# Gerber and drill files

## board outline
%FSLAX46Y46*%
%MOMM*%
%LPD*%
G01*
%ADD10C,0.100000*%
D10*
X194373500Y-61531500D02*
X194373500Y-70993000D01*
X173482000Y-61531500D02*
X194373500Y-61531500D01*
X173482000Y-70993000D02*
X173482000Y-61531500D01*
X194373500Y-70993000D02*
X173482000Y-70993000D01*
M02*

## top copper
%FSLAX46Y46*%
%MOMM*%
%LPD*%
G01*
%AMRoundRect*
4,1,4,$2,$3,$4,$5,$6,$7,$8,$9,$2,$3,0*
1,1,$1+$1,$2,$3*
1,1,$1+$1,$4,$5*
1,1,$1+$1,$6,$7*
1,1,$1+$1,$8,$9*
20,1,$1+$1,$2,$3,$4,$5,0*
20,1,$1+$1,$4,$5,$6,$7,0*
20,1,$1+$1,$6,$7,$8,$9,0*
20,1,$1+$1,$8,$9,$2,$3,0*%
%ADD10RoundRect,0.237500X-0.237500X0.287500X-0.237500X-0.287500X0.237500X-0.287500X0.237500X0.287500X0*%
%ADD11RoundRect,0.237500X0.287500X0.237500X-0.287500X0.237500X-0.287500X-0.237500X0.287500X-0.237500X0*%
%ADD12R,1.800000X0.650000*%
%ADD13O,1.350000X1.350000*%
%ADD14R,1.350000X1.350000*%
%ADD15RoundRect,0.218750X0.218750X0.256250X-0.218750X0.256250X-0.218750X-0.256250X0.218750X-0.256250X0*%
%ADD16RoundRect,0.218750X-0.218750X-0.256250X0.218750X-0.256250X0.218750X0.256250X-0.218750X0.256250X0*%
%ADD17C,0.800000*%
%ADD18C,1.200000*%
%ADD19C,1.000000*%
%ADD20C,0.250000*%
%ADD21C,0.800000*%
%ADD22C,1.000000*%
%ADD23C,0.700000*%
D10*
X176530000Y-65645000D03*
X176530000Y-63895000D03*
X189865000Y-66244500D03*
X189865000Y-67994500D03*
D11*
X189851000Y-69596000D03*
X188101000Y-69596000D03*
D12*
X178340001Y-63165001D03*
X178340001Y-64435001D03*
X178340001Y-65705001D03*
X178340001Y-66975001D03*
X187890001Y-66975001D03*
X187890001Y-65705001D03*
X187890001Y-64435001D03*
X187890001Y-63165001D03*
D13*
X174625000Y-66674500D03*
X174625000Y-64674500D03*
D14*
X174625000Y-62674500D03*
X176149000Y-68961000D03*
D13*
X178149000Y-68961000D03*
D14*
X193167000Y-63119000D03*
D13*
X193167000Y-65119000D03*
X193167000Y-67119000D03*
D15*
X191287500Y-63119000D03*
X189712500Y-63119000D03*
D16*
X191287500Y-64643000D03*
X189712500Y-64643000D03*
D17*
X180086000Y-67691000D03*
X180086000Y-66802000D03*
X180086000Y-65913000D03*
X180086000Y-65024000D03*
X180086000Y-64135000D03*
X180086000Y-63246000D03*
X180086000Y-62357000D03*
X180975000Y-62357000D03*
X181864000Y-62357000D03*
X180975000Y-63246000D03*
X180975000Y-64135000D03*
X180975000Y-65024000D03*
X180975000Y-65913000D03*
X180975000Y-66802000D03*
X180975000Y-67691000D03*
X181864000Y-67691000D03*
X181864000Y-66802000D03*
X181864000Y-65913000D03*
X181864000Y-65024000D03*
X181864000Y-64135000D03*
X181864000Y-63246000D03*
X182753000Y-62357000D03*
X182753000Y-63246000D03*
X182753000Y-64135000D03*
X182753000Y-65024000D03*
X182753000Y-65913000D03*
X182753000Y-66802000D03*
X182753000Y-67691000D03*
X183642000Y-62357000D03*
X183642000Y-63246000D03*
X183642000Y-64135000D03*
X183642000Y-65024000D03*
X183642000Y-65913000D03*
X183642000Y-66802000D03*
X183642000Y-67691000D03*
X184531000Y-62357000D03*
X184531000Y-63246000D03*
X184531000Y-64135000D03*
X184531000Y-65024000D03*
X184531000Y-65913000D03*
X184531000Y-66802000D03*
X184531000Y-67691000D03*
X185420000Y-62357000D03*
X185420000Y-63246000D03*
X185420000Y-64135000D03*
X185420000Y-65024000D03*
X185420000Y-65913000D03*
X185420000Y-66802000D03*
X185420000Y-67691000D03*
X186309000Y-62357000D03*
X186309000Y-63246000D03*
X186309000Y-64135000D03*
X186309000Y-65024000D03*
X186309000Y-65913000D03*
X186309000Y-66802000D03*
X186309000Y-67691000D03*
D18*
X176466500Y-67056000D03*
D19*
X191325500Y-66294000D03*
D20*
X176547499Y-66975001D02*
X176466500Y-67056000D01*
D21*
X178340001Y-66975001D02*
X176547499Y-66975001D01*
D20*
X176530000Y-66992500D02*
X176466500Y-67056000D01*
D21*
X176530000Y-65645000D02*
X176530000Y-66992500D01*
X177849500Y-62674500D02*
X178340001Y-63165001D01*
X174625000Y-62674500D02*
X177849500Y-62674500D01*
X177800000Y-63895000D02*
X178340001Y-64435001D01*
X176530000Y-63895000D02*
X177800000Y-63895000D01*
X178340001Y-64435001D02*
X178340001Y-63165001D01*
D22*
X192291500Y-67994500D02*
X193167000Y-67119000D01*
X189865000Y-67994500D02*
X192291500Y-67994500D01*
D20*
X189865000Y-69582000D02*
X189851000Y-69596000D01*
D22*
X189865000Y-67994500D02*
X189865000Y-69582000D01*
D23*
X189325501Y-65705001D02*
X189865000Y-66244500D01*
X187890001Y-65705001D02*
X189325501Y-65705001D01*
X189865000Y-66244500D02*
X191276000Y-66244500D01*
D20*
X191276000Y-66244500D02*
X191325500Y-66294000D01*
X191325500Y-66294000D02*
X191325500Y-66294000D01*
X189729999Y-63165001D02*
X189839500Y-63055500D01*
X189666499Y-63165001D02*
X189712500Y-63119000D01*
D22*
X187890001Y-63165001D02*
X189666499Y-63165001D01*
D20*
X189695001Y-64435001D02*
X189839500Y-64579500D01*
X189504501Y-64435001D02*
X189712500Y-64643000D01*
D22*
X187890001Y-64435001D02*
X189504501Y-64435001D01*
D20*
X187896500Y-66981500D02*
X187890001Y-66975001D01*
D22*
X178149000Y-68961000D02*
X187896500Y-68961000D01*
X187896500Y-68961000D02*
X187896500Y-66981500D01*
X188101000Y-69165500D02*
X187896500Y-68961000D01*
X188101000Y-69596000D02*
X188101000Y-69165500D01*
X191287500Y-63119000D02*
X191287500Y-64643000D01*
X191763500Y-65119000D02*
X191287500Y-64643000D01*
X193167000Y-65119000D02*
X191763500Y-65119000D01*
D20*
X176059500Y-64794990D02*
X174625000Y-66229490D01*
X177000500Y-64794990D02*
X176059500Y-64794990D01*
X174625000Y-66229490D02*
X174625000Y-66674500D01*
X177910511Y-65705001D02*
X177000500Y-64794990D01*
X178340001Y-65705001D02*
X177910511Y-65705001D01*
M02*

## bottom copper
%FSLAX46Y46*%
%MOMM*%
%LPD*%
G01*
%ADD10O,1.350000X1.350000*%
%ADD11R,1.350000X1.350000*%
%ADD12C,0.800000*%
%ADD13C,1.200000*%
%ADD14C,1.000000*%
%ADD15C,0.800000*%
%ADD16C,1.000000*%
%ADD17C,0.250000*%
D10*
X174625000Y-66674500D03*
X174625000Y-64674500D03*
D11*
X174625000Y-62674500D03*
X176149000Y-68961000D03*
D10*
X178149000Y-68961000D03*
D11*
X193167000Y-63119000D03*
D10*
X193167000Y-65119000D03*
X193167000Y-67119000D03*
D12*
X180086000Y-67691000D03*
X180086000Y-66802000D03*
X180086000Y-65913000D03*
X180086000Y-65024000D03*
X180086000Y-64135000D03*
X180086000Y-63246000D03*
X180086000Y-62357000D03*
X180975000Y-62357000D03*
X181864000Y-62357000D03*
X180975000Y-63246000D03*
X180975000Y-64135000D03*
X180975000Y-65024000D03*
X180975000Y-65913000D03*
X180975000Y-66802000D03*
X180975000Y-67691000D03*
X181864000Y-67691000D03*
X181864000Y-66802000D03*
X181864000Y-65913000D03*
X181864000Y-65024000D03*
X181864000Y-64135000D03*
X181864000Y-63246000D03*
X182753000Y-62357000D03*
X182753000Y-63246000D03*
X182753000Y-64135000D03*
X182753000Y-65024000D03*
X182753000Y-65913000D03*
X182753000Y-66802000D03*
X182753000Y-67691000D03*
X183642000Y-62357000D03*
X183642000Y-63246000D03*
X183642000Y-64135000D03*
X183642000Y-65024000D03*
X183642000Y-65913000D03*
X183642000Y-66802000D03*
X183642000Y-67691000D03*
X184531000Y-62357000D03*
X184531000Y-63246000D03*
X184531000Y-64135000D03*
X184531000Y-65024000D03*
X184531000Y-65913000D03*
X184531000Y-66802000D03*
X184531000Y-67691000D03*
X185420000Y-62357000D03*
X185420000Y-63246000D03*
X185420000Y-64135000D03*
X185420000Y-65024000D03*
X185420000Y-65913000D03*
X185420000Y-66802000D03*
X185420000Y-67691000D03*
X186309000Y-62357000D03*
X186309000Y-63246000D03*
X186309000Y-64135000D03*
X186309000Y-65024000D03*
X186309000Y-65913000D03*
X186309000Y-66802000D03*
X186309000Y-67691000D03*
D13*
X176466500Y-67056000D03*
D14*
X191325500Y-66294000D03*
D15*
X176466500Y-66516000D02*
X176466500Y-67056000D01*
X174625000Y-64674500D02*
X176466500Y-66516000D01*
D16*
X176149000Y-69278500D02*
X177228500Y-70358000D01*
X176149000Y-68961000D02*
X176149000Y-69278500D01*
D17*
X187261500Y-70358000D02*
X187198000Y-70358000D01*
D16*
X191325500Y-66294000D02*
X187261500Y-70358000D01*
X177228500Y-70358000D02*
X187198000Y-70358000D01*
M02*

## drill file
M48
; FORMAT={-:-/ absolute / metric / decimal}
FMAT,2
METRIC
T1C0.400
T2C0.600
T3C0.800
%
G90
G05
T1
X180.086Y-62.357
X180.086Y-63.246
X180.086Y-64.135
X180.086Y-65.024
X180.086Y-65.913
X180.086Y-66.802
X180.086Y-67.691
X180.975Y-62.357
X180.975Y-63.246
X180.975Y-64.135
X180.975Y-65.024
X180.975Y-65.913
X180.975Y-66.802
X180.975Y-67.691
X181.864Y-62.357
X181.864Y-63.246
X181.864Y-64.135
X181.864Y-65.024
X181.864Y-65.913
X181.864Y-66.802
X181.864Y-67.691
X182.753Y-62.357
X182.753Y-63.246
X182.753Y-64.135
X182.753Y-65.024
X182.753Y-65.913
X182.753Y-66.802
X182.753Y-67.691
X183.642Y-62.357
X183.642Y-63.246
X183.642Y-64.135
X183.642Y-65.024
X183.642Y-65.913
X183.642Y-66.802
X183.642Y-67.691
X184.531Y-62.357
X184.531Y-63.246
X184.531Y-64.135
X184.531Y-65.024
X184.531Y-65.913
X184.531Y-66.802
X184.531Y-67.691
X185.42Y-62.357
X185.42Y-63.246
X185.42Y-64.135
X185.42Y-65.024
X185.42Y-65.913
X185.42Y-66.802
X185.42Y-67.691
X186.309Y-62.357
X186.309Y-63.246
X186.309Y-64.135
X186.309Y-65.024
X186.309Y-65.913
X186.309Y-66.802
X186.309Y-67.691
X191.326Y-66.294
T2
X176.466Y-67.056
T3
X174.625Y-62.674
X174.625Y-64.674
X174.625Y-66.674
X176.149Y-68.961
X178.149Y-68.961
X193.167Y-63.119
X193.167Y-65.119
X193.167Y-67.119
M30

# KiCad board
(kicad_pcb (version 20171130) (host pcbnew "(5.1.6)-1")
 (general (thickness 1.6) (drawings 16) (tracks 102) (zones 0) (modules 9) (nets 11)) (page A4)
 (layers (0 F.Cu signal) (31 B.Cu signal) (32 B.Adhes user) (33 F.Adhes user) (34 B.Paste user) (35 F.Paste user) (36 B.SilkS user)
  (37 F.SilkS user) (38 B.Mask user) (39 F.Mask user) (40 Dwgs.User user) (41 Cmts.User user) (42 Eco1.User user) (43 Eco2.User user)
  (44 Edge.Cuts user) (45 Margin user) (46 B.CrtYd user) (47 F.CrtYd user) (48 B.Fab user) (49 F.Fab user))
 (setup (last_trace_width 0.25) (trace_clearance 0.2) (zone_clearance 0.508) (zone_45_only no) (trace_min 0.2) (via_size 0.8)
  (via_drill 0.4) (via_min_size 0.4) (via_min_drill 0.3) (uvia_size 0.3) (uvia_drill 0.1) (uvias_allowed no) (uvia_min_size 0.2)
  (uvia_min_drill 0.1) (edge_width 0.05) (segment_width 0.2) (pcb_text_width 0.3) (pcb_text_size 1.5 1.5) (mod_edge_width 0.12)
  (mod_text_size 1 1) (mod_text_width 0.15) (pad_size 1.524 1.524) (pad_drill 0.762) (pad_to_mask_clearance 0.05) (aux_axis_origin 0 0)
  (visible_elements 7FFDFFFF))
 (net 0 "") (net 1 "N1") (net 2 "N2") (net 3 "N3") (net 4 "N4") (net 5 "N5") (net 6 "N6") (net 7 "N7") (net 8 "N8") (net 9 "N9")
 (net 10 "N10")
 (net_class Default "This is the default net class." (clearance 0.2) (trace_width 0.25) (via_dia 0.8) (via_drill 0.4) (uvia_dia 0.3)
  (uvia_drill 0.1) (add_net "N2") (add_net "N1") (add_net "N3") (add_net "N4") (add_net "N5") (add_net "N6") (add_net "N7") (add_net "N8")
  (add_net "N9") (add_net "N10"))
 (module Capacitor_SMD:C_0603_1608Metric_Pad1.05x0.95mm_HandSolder (layer F.Cu) (at 176.53 64.77 270)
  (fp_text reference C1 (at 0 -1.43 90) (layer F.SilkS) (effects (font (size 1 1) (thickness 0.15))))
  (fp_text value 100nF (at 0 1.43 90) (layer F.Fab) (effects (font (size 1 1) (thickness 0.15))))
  (pad 2 smd roundrect (at 0.875 0 270) (size 1.05 0.95) (layers F.Cu F.Paste F.Mask) (roundrect_rratio 0.25) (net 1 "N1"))
  (pad 1 smd roundrect (at -0.875 0 270) (size 1.05 0.95) (layers F.Cu F.Paste F.Mask) (roundrect_rratio 0.25) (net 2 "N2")))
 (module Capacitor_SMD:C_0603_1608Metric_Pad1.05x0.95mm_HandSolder (layer F.Cu) (at 189.865 67.1195 270)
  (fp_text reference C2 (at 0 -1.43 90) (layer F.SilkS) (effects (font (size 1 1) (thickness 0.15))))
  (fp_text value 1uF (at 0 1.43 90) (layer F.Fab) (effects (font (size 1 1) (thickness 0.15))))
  (pad 1 smd roundrect (at -0.875 0 270) (size 1.05 0.95) (layers F.Cu F.Paste F.Mask) (roundrect_rratio 0.25) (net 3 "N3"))
  (pad 2 smd roundrect (at 0.875 0 270) (size 1.05 0.95) (layers F.Cu F.Paste F.Mask) (roundrect_rratio 0.25) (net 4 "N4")))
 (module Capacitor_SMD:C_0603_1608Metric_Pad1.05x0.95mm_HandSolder (layer F.Cu) (at 188.976 69.596 180)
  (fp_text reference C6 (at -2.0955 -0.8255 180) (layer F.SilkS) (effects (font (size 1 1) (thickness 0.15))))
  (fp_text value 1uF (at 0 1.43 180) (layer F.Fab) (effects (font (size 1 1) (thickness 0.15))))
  (pad 1 smd roundrect (at -0.875 0 180) (size 1.05 0.95) (layers F.Cu F.Paste F.Mask) (roundrect_rratio 0.25) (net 4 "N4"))
  (pad 2 smd roundrect (at 0.875 0 180) (size 1.05 0.95) (layers F.Cu F.Paste F.Mask) (roundrect_rratio 0.25) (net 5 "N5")))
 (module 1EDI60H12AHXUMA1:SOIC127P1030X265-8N (layer F.Cu) (at 183.115001 65.070001)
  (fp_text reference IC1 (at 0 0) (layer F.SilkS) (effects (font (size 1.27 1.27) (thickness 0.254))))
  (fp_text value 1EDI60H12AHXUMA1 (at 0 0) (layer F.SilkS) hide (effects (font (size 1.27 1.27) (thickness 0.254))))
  (pad 1 smd rect (at -4.775 -1.905 90) (size 0.65 1.8) (layers F.Cu F.Paste F.Mask) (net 2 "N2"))
  (pad 2 smd rect (at -4.775 -0.635 90) (size 0.65 1.8) (layers F.Cu F.Paste F.Mask) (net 2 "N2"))
  (pad 3 smd rect (at -4.775 0.635 90) (size 0.65 1.8) (layers F.Cu F.Paste F.Mask) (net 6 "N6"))
  (pad 4 smd rect (at -4.775 1.905 90) (size 0.65 1.8) (layers F.Cu F.Paste F.Mask) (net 1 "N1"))
  (pad 5 smd rect (at 4.775 1.905 90) (size 0.65 1.8) (layers F.Cu F.Paste F.Mask) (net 5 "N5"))
  (pad 6 smd rect (at 4.775 0.635 90) (size 0.65 1.8) (layers F.Cu F.Paste F.Mask) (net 3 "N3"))
  (pad 7 smd rect (at 4.775 -0.635 90) (size 0.65 1.8) (layers F.Cu F.Paste F.Mask) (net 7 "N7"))
  (pad 8 smd rect (at 4.775 -1.905 90) (size 0.65 1.8) (layers F.Cu F.Paste F.Mask) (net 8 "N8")))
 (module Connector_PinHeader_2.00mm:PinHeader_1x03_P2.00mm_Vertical (layer B.Cu) (at 174.625 62.6745 180)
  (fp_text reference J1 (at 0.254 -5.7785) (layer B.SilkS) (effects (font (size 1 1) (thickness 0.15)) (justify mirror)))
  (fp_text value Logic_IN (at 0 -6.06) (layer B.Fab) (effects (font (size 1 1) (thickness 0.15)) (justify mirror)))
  (pad 3 thru_hole oval (at 0 -4 180) (size 1.35 1.35) (drill 0.8) (layers *.Cu *.Mask) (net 6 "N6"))
  (pad 2 thru_hole oval (at 0 -2 180) (size 1.35 1.35) (drill 0.8) (layers *.Cu *.Mask) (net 1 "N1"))
  (pad 1 thru_hole rect (at 0 0 180) (size 1.35 1.35) (drill 0.8) (layers *.Cu *.Mask) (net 2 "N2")))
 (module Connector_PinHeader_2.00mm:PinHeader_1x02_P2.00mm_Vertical (layer B.Cu) (at 176.149 68.961 270)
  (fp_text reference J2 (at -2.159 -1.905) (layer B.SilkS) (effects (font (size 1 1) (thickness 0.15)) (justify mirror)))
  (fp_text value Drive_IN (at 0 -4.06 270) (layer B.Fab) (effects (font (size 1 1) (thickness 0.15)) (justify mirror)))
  (pad 1 thru_hole rect (at 0 0 270) (size 1.35 1.35) (drill 0.8) (layers *.Cu *.Mask) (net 3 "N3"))
  (pad 2 thru_hole oval (at 0 -2 270) (size 1.35 1.35) (drill 0.8) (layers *.Cu *.Mask) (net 5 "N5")))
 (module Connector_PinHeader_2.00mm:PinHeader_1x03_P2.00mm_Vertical (layer B.Cu) (at 193.167 63.119 180)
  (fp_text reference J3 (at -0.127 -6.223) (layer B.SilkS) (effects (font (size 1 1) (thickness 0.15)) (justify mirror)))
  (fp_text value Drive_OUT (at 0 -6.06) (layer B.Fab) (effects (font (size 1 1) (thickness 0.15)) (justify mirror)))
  (pad 1 thru_hole rect (at 0 0 180) (size 1.35 1.35) (drill 0.8) (layers *.Cu *.Mask) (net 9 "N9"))
  (pad 2 thru_hole oval (at 0 -2 180) (size 1.35 1.35) (drill 0.8) (layers *.Cu *.Mask) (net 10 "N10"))
  (pad 3 thru_hole oval (at 0 -4 180) (size 1.35 1.35) (drill 0.8) (layers *.Cu *.Mask) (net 4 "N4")))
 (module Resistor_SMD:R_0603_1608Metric (layer F.Cu) (at 190.5 63.119 180)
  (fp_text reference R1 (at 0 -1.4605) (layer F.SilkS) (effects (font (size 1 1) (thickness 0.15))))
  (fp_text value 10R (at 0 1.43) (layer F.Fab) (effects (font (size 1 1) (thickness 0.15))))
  (pad 1 smd roundrect (at -0.7875 0 180) (size 0.875 0.95) (layers F.Cu F.Paste F.Mask) (roundrect_rratio 0.25) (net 10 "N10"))
  (pad 2 smd roundrect (at 0.7875 0 180) (size 0.875 0.95) (layers F.Cu F.Paste F.Mask) (roundrect_rratio 0.25) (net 8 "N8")))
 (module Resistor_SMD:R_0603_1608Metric (layer F.Cu) (at 190.5 64.643)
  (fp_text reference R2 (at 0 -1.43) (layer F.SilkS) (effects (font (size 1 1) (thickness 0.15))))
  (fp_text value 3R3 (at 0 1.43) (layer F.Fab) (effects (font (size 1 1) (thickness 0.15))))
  (pad 2 smd roundrect (at 0.7875 0) (size 0.875 0.95) (layers F.Cu F.Paste F.Mask) (roundrect_rratio 0.25) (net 10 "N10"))
  (pad 1 smd roundrect (at -0.7875 0) (size 0.875 0.95) (layers F.Cu F.Paste F.Mask) (roundrect_rratio 0.25) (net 7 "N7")))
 (gr_line (start 194.3735 61.5315) (end 194.3735 70.993) (layer Edge.Cuts) (width 0.1))
 (gr_line (start 173.482 61.5315) (end 194.3735 61.5315) (layer Edge.Cuts) (width 0.1))
 (gr_line (start 173.482 70.993) (end 173.482 61.5315) (layer Edge.Cuts) (width 0.1))
 (gr_line (start 194.3735 70.993) (end 173.482 70.993) (layer Edge.Cuts) (width 0.1))
 (via (at 180.086 67.691) (size 0.8) (drill 0.4) (layers F.Cu B.Cu) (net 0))
 (via (at 180.086 66.802) (size 0.8) (drill 0.4) (layers F.Cu B.Cu) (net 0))
 (via (at 180.086 65.913) (size 0.8) (drill 0.4) (layers F.Cu B.Cu) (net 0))
 (via (at 180.086 65.024) (size 0.8) (drill 0.4) (layers F.Cu B.Cu) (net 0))
 (via (at 180.086 64.135) (size 0.8) (drill 0.4) (layers F.Cu B.Cu) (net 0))
 (via (at 180.086 63.246) (size 0.8) (drill 0.4) (layers F.Cu B.Cu) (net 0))
 (via (at 180.086 62.357) (size 0.8) (drill 0.4) (layers F.Cu B.Cu) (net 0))
 (via (at 180.975 62.357) (size 0.8) (drill 0.4) (layers F.Cu B.Cu) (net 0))
 (via (at 181.864 62.357) (size 0.8) (drill 0.4) (layers F.Cu B.Cu) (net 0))
 (via (at 180.975 63.246) (size 0.8) (drill 0.4) (layers F.Cu B.Cu) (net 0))
 (via (at 180.975 64.135) (size 0.8) (drill 0.4) (layers F.Cu B.Cu) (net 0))
 (via (at 180.975 65.024) (size 0.8) (drill 0.4) (layers F.Cu B.Cu) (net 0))
 (via (at 180.975 65.913) (size 0.8) (drill 0.4) (layers F.Cu B.Cu) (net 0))
 (via (at 180.975 66.802) (size 0.8) (drill 0.4) (layers F.Cu B.Cu) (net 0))
 (via (at 180.975 67.691) (size 0.8) (drill 0.4) (layers F.Cu B.Cu) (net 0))
 (via (at 181.864 67.691) (size 0.8) (drill 0.4) (layers F.Cu B.Cu) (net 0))
 (via (at 181.864 66.802) (size 0.8) (drill 0.4) (layers F.Cu B.Cu) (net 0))
 (via (at 181.864 65.913) (size 0.8) (drill 0.4) (layers F.Cu B.Cu) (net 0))
 (via (at 181.864 65.024) (size 0.8) (drill 0.4) (layers F.Cu B.Cu) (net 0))
 (via (at 181.864 64.135) (size 0.8) (drill 0.4) (layers F.Cu B.Cu) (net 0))
 (via (at 181.864 63.246) (size 0.8) (drill 0.4) (layers F.Cu B.Cu) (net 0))
 (via (at 182.753 62.357) (size 0.8) (drill 0.4) (layers F.Cu B.Cu) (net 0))
 (via (at 182.753 63.246) (size 0.8) (drill 0.4) (layers F.Cu B.Cu) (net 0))
 (via (at 182.753 64.135) (size 0.8) (drill 0.4) (layers F.Cu B.Cu) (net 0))
 (via (at 182.753 65.024) (size 0.8) (drill 0.4) (layers F.Cu B.Cu) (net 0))
 (via (at 182.753 65.913) (size 0.8) (drill 0.4) (layers F.Cu B.Cu) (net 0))
 (via (at 182.753 66.802) (size 0.8) (drill 0.4) (layers F.Cu B.Cu) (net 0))
 (via (at 182.753 67.691) (size 0.8) (drill 0.4) (layers F.Cu B.Cu) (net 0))
 (via (at 183.642 62.357) (size 0.8) (drill 0.4) (layers F.Cu B.Cu) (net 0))
 (via (at 183.642 63.246) (size 0.8) (drill 0.4) (layers F.Cu B.Cu) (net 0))
 (via (at 183.642 64.135) (size 0.8) (drill 0.4) (layers F.Cu B.Cu) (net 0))
 (via (at 183.642 65.024) (size 0.8) (drill 0.4) (layers F.Cu B.Cu) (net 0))
 (via (at 183.642 65.913) (size 0.8) (drill 0.4) (layers F.Cu B.Cu) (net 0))
 (via (at 183.642 66.802) (size 0.8) (drill 0.4) (layers F.Cu B.Cu) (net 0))
 (via (at 183.642 67.691) (size 0.8) (drill 0.4) (layers F.Cu B.Cu) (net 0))
 (via (at 184.531 62.357) (size 0.8) (drill 0.4) (layers F.Cu B.Cu) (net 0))
 (via (at 184.531 63.246) (size 0.8) (drill 0.4) (layers F.Cu B.Cu) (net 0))
 (via (at 184.531 64.135) (size 0.8) (drill 0.4) (layers F.Cu B.Cu) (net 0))
 (via (at 184.531 65.024) (size 0.8) (drill 0.4) (layers F.Cu B.Cu) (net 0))
 (via (at 184.531 65.913) (size 0.8) (drill 0.4) (layers F.Cu B.Cu) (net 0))
 (via (at 184.531 66.802) (size 0.8) (drill 0.4) (layers F.Cu B.Cu) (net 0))
 (via (at 184.531 67.691) (size 0.8) (drill 0.4) (layers F.Cu B.Cu) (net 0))
 (via (at 185.42 62.357) (size 0.8) (drill 0.4) (layers F.Cu B.Cu) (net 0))
 (via (at 185.42 63.246) (size 0.8) (drill 0.4) (layers F.Cu B.Cu) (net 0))
 (via (at 185.42 64.135) (size 0.8) (drill 0.4) (layers F.Cu B.Cu) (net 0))
 (via (at 185.42 65.024) (size 0.8) (drill 0.4) (layers F.Cu B.Cu) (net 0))
 (via (at 185.42 65.913) (size 0.8) (drill 0.4) (layers F.Cu B.Cu) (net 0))
 (via (at 185.42 66.802) (size 0.8) (drill 0.4) (layers F.Cu B.Cu) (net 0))
 (via (at 185.42 67.691) (size 0.8) (drill 0.4) (layers F.Cu B.Cu) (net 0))
 (via (at 186.309 62.357) (size 0.8) (drill 0.4) (layers F.Cu B.Cu) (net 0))
 (via (at 186.309 63.246) (size 0.8) (drill 0.4) (layers F.Cu B.Cu) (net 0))
 (via (at 186.309 64.135) (size 0.8) (drill 0.4) (layers F.Cu B.Cu) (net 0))
 (via (at 186.309 65.024) (size 0.8) (drill 0.4) (layers F.Cu B.Cu) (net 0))
 (via (at 186.309 65.913) (size 0.8) (drill 0.4) (layers F.Cu B.Cu) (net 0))
 (via (at 186.309 66.802) (size 0.8) (drill 0.4) (layers F.Cu B.Cu) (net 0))
 (via (at 186.309 67.691) (size 0.8) (drill 0.4) (layers F.Cu B.Cu) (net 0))
 (via (at 176.4665 67.056) (size 1.2) (drill 0.6) (layers F.Cu B.Cu) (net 1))
 (segment (start 176.547499 66.975001) (end 176.4665 67.056) (width 0.25) (layer F.Cu) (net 1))
 (segment (start 178.340001 66.975001) (end 176.547499 66.975001) (width 0.8) (layer F.Cu) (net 1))
 (segment (start 176.53 66.9925) (end 176.4665 67.056) (width 0.25) (layer F.Cu) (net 1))
 (segment (start 176.53 65.645) (end 176.53 66.9925) (width 0.8) (layer F.Cu) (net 1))
 (segment (start 176.4665 66.516) (end 176.4665 67.056) (width 0.8) (layer B.Cu) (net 1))
 (segment (start 174.625 64.6745) (end 176.4665 66.516) (width 0.8) (layer B.Cu) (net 1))
 (segment (start 177.8495 62.6745) (end 178.340001 63.165001) (width 0.8) (layer F.Cu) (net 2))
 (segment (start 174.625 62.6745) (end 177.8495 62.6745) (width 0.8) (layer F.Cu) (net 2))
 (segment (start 177.8 63.895) (end 178.340001 64.435001) (width 0.8) (layer F.Cu) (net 2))
 (segment (start 176.53 63.895) (end 177.8 63.895) (width 0.8) (layer F.Cu) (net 2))
 (segment (start 178.340001 64.435001) (end 178.340001 63.165001) (width 0.8) (layer F.Cu) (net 2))
 (segment (start 192.2915 67.9945) (end 193.167 67.119) (width 1) (layer F.Cu) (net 4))
 (segment (start 189.865 67.9945) (end 192.2915 67.9945) (width 1) (layer F.Cu) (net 4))
 (segment (start 189.865 69.582) (end 189.851 69.596) (width 0.25) (layer F.Cu) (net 4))
 (segment (start 189.865 67.9945) (end 189.865 69.582) (width 1) (layer F.Cu) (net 4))
 (segment (start 189.325501 65.705001) (end 189.865 66.2445) (width 0.7) (layer F.Cu) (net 3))
 (segment (start 187.890001 65.705001) (end 189.325501 65.705001) (width 0.7) (layer F.Cu) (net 3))
 (segment (start 189.865 66.2445) (end 191.276 66.2445) (width 0.7) (layer F.Cu) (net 3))
 (segment (start 191.276 66.2445) (end 191.3255 66.294) (width 0.25) (layer F.Cu) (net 3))
 (segment (start 191.3255 66.294) (end 191.3255 66.294) (width 0.25) (layer F.Cu) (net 3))
 (via (at 191.3255 66.294) (size 1) (drill 0.4) (layers F.Cu B.Cu) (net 3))
 (segment (start 176.149 69.2785) (end 177.2285 70.358) (width 1) (layer B.Cu) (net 3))
 (segment (start 176.149 68.961) (end 176.149 69.2785) (width 1) (layer B.Cu) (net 3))
 (segment (start 187.2615 70.358) (end 187.198 70.358) (width 0.25) (layer B.Cu) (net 3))
 (segment (start 191.3255 66.294) (end 187.2615 70.358) (width 1) (layer B.Cu) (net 3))
 (segment (start 177.2285 70.358) (end 187.198 70.358) (width 1) (layer B.Cu) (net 3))
 (segment (start 189.729999 63.165001) (end 189.8395 63.0555) (width 0.25) (layer F.Cu) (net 8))
 (segment (start 189.666499 63.165001) (end 189.7125 63.119) (width 0.25) (layer F.Cu) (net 8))
 (segment (start 187.890001 63.165001) (end 189.666499 63.165001) (width 1) (layer F.Cu) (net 8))
 (segment (start 189.695001 64.435001) (end 189.8395 64.5795) (width 0.25) (layer F.Cu) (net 7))
 (segment (start 189.504501 64.435001) (end 189.7125 64.643) (width 0.25) (layer F.Cu) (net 7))
 (segment (start 187.890001 64.435001) (end 189.504501 64.435001) (width 1) (layer F.Cu) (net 7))
 (segment (start 187.8965 66.9815) (end 187.890001 66.975001) (width 0.25) (layer F.Cu) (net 5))
 (segment (start 178.149 68.961) (end 187.8965 68.961) (width 1) (layer F.Cu) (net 5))
 (segment (start 187.8965 68.961) (end 187.8965 66.9815) (width 1) (layer F.Cu) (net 5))
 (segment (start 188.101 69.1655) (end 187.8965 68.961) (width 1) (layer F.Cu) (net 5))
 (segment (start 188.101 69.596) (end 188.101 69.1655) (width 1) (layer F.Cu) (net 5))
 (segment (start 191.2875 63.119) (end 191.2875 64.643) (width 1) (layer F.Cu) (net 10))
 (segment (start 191.7635 65.119) (end 191.2875 64.643) (width 1) (layer F.Cu) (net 10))
 (segment (start 193.167 65.119) (end 191.7635 65.119) (width 1) (layer F.Cu) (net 10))
 (segment (start 176.0595 64.79499) (end 174.625 66.22949) (width 0.25) (layer F.Cu) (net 6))
 (segment (start 177.0005 64.79499) (end 176.0595 64.79499) (width 0.25) (layer F.Cu) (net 6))
 (segment (start 174.625 66.22949) (end 174.625 66.6745) (width 0.25) (layer F.Cu) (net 6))
 (segment (start 177.910511 65.705001) (end 177.0005 64.79499) (width 0.25) (layer F.Cu) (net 6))
 (segment (start 178.340001 65.705001) (end 177.910511 65.705001) (width 0.25) (layer F.Cu) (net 6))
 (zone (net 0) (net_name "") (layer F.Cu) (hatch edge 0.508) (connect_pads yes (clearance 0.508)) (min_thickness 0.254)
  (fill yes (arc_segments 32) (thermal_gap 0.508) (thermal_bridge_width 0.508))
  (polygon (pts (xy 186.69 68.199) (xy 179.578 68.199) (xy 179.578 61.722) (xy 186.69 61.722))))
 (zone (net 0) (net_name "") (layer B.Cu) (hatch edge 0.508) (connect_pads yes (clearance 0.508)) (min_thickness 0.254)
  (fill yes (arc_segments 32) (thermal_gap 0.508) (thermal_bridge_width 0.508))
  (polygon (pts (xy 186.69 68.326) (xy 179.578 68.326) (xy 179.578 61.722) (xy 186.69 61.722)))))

